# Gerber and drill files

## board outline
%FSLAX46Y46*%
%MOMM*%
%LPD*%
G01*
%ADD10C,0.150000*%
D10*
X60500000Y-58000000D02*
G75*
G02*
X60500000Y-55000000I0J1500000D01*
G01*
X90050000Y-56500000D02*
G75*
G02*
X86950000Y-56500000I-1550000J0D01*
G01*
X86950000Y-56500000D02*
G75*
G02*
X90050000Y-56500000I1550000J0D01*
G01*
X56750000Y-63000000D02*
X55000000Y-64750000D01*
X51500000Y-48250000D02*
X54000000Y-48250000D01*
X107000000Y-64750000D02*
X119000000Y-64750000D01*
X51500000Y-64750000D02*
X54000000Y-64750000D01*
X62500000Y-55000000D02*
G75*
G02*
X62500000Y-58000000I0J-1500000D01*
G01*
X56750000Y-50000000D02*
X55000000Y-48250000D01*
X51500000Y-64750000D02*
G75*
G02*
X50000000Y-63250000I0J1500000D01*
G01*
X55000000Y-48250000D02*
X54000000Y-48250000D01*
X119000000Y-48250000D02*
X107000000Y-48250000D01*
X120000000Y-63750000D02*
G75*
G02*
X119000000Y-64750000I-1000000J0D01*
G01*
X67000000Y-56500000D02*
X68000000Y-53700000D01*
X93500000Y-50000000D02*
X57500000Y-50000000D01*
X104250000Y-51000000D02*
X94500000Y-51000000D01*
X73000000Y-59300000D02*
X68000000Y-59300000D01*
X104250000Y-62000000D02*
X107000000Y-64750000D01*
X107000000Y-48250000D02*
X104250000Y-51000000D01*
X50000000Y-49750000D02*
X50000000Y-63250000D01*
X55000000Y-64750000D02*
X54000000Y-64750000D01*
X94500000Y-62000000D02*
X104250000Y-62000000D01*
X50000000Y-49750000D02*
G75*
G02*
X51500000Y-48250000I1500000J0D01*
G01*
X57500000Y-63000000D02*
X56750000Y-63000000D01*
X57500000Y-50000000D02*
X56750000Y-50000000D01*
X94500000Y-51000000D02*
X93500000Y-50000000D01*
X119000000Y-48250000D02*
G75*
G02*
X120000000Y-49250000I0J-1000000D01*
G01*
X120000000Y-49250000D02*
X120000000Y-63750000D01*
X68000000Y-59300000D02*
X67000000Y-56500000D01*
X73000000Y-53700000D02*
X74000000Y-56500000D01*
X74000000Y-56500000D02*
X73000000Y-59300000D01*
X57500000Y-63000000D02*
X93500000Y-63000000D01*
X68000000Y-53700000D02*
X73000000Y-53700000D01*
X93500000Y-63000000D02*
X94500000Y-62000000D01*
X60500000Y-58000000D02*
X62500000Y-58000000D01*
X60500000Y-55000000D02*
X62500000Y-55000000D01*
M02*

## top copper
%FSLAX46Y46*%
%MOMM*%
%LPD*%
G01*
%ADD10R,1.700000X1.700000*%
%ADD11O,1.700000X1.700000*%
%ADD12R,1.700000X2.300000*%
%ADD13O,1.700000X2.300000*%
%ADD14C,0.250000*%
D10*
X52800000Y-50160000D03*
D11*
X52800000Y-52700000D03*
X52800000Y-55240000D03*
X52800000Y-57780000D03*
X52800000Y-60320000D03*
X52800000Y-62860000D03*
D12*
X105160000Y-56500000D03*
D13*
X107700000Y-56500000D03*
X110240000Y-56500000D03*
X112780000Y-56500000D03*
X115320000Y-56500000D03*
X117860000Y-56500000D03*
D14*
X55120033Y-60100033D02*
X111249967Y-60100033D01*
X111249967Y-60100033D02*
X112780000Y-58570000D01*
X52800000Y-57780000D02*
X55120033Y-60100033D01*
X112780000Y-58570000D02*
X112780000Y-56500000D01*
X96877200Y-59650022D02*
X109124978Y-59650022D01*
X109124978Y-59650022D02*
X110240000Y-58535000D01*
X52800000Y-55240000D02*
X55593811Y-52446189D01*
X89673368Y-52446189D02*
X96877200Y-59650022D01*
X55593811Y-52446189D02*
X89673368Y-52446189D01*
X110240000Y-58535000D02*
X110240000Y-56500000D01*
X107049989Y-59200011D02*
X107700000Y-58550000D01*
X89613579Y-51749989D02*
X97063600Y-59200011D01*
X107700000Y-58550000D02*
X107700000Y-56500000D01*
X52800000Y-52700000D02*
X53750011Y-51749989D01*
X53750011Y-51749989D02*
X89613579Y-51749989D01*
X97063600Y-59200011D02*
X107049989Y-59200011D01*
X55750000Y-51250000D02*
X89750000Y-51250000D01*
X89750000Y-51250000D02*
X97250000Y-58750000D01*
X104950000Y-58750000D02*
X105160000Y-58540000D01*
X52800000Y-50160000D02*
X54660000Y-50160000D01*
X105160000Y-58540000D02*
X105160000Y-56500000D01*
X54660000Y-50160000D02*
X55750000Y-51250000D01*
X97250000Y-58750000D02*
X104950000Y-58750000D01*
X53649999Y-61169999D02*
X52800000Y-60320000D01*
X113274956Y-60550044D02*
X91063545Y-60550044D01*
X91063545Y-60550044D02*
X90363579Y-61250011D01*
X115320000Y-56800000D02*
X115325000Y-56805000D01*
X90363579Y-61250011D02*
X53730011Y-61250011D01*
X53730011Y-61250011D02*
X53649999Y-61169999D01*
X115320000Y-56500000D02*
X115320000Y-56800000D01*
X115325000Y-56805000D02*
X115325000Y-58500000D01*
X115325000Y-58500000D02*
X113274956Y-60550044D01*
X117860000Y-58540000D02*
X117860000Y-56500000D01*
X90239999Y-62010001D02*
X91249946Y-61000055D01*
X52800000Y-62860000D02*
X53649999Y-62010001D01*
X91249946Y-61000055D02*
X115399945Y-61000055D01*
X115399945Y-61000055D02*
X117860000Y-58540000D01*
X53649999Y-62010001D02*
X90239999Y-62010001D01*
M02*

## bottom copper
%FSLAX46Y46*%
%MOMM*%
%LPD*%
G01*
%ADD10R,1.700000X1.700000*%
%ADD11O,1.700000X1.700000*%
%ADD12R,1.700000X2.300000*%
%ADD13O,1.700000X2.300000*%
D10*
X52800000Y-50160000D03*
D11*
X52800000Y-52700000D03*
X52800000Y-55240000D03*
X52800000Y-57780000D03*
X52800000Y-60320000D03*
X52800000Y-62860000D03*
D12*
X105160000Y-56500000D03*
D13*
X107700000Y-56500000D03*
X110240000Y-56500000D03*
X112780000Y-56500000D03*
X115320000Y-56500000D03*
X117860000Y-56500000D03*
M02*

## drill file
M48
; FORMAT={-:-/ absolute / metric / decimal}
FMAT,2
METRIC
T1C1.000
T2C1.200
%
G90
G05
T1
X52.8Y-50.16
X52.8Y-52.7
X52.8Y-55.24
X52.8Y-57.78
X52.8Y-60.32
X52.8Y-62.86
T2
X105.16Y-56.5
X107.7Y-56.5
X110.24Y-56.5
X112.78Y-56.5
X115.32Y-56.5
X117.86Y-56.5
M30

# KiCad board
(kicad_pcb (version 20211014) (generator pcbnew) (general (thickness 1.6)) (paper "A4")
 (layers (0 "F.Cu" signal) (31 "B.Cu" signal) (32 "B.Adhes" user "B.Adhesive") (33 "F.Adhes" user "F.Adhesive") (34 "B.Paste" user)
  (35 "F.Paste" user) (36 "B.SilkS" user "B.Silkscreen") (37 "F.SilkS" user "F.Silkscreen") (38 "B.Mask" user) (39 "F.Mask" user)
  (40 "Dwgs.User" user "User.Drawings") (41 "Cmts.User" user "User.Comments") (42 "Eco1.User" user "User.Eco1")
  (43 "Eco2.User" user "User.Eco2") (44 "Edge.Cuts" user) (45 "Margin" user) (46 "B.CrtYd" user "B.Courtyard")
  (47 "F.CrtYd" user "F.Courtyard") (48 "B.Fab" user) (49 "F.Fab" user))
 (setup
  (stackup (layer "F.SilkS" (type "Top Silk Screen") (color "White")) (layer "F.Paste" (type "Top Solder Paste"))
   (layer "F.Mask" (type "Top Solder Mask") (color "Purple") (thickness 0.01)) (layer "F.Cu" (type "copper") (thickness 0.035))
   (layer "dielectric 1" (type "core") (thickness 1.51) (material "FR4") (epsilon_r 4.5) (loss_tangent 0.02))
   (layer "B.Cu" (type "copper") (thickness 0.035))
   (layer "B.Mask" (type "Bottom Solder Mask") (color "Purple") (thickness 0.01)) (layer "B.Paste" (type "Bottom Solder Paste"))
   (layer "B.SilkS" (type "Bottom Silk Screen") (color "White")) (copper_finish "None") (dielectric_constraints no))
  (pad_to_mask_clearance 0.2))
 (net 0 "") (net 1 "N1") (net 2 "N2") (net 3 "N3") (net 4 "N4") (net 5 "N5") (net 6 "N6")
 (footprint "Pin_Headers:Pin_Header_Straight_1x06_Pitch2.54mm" (layer "F.Cu") (at 52.8 50.16)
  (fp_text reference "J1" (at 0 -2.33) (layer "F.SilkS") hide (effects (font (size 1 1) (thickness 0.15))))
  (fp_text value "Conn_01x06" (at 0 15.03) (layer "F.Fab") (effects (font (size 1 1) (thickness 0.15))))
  (pad "1" thru_hole rect locked (at 0 0) (size 1.7 1.7) (drill 1) (layers *.Cu *.Mask) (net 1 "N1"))
  (pad "2" thru_hole oval locked (at 0 2.54) (size 1.7 1.7) (drill 1) (layers *.Cu *.Mask) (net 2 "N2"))
  (pad "3" thru_hole oval locked (at 0 5.08) (size 1.7 1.7) (drill 1) (layers *.Cu *.Mask) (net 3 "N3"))
  (pad "4" thru_hole oval locked (at 0 7.62) (size 1.7 1.7) (drill 1) (layers *.Cu *.Mask) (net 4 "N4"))
  (pad "5" thru_hole oval locked (at 0 10.16) (size 1.7 1.7) (drill 1) (layers *.Cu *.Mask) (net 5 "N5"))
  (pad "6" thru_hole oval locked (at 0 12.7) (size 1.7 1.7) (drill 1) (layers *.Cu *.Mask) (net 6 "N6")))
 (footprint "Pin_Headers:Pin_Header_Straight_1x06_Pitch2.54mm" (layer "F.Cu") (at 105.16 56.5 90)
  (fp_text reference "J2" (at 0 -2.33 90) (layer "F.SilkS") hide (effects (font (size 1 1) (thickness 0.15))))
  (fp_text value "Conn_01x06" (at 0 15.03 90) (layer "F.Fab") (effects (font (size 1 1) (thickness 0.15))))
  (pad "1" thru_hole rect locked (at 0 0 90) (size 2.3 1.7) (drill 1.2) (layers *.Cu *.Mask) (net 1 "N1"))
  (pad "2" thru_hole oval locked (at 0 2.54 90) (size 2.3 1.7) (drill 1.2) (layers *.Cu *.Mask) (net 2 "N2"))
  (pad "3" thru_hole oval locked (at 0 5.08 90) (size 2.3 1.7) (drill 1.2) (layers *.Cu *.Mask) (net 3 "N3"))
  (pad "4" thru_hole oval locked (at 0 7.62 90) (size 2.3 1.7) (drill 1.2) (layers *.Cu *.Mask) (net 4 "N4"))
  (pad "5" thru_hole oval locked (at 0 10.16 90) (size 2.3 1.7) (drill 1.2) (layers *.Cu *.Mask) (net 5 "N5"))
  (pad "6" thru_hole oval locked (at 0 12.7 90) (size 2.3 1.7) (drill 1.2) (layers *.Cu *.Mask) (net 6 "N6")))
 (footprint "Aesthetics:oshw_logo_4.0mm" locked (layer "F.Cu") (at 99.695 56.515 -90)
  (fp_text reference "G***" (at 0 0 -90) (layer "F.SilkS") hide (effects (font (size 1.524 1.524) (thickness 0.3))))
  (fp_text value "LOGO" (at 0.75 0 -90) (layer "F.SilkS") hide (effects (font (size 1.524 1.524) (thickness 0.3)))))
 (gr_arc (start 60.5 58) (mid 59 56.5) (end 60.5 55) (layer "Edge.Cuts") (width 0.15))
 (gr_arc (start 90.05 56.5) (mid 88.5 58.05) (end 86.95 56.5) (layer "Edge.Cuts") (width 0.15))
 (gr_arc (start 86.95 56.5) (mid 88.5 54.95) (end 90.05 56.5) (layer "Edge.Cuts") (width 0.15))
 (gr_line (start 56.75 63) (end 55 64.75) (layer "Edge.Cuts") (width 0.15))
 (gr_line (start 51.5 48.25) (end 54 48.25) (layer "Edge.Cuts") (width 0.15))
 (gr_line (start 107 64.75) (end 119 64.75) (layer "Edge.Cuts") (width 0.15))
 (gr_line (start 51.5 64.75) (end 54 64.75) (layer "Edge.Cuts") (width 0.15))
 (gr_arc (start 62.5 55) (mid 64 56.5) (end 62.5 58) (layer "Edge.Cuts") (width 0.15))
 (gr_line (start 56.75 50) (end 55 48.25) (layer "Edge.Cuts") (width 0.15))
 (gr_arc (start 51.5 64.75) (mid 50.43934 64.31066) (end 50 63.25) (layer "Edge.Cuts") (width 0.15))
 (gr_line (start 55 48.25) (end 54 48.25) (layer "Edge.Cuts") (width 0.15))
 (gr_line (start 119 48.25) (end 107 48.25) (layer "Edge.Cuts") (width 0.15))
 (gr_arc (start 120 63.75) (mid 119.707107 64.457107) (end 119 64.75) (layer "Edge.Cuts") (width 0.15))
 (gr_line (start 67 56.5) (end 68 53.7) (layer "Edge.Cuts") (width 0.15))
 (gr_line (start 93.5 50) (end 57.5 50) (layer "Edge.Cuts") (width 0.15))
 (gr_line (start 104.25 51) (end 94.5 51) (layer "Edge.Cuts") (width 0.15))
 (gr_line (start 73 59.3) (end 68 59.3) (layer "Edge.Cuts") (width 0.15))
 (gr_line (start 104.25 62) (end 107 64.75) (layer "Edge.Cuts") (width 0.15))
 (gr_line (start 107 48.25) (end 104.25 51) (layer "Edge.Cuts") (width 0.15))
 (gr_line (start 50 49.75) (end 50 63.25) (layer "Edge.Cuts") (width 0.15))
 (gr_line (start 55 64.75) (end 54 64.75) (layer "Edge.Cuts") (width 0.15))
 (gr_line (start 94.5 62) (end 104.25 62) (layer "Edge.Cuts") (width 0.15))
 (gr_arc (start 50 49.75) (mid 50.43934 48.68934) (end 51.5 48.25) (layer "Edge.Cuts") (width 0.15))
 (gr_line (start 57.5 63) (end 56.75 63) (layer "Edge.Cuts") (width 0.15))
 (gr_line (start 57.5 50) (end 56.75 50) (layer "Edge.Cuts") (width 0.15))
 (gr_line (start 94.5 51) (end 93.5 50) (layer "Edge.Cuts") (width 0.15))
 (gr_arc (start 119 48.25) (mid 119.707107 48.542893) (end 120 49.25) (layer "Edge.Cuts") (width 0.15))
 (gr_line (start 120 49.25) (end 120 63.75) (layer "Edge.Cuts") (width 0.15))
 (gr_line (start 68 59.3) (end 67 56.5) (layer "Edge.Cuts") (width 0.15))
 (gr_line (start 73 53.7) (end 74 56.5) (layer "Edge.Cuts") (width 0.15))
 (gr_line (start 74 56.5) (end 73 59.3) (layer "Edge.Cuts") (width 0.15))
 (gr_line (start 57.5 63) (end 93.5 63) (layer "Edge.Cuts") (width 0.15))
 (gr_line (start 68 53.7) (end 73 53.7) (layer "Edge.Cuts") (width 0.15))
 (gr_line (start 93.5 63) (end 94.5 62) (layer "Edge.Cuts") (width 0.15))
 (gr_line (start 60.5 58) (end 62.5 58) (layer "Edge.Cuts") (width 0.15))
 (gr_line (start 60.5 55) (end 62.5 55) (layer "Edge.Cuts") (width 0.15))
 (segment (start 55.120033 60.100033) (end 111.249967 60.100033) (width 0.25) (layer "F.Cu") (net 4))
 (segment (start 111.249967 60.100033) (end 112.78 58.57) (width 0.25) (layer "F.Cu") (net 4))
 (segment (start 52.8 57.78) (end 55.120033 60.100033) (width 0.25) (layer "F.Cu") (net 4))
 (segment (start 112.78 58.57) (end 112.78 56.5) (width 0.25) (layer "F.Cu") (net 4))
 (segment (start 96.8772 59.650022) (end 109.124978 59.650022) (width 0.25) (layer "F.Cu") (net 3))
 (segment (start 109.124978 59.650022) (end 110.24 58.535) (width 0.25) (layer "F.Cu") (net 3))
 (segment (start 52.8 55.24) (end 55.593811 52.446189) (width 0.25) (layer "F.Cu") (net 3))
 (segment (start 89.673368 52.446189) (end 96.8772 59.650022) (width 0.25) (layer "F.Cu") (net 3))
 (segment (start 55.593811 52.446189) (end 89.673368 52.446189) (width 0.25) (layer "F.Cu") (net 3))
 (segment (start 110.24 58.535) (end 110.24 56.5) (width 0.25) (layer "F.Cu") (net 3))
 (segment (start 107.049989 59.200011) (end 107.7 58.55) (width 0.25) (layer "F.Cu") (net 2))
 (segment (start 89.613579 51.749989) (end 97.0636 59.200011) (width 0.25) (layer "F.Cu") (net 2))
 (segment (start 107.7 58.55) (end 107.7 56.5) (width 0.25) (layer "F.Cu") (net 2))
 (segment (start 52.8 52.7) (end 53.750011 51.749989) (width 0.25) (layer "F.Cu") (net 2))
 (segment (start 53.750011 51.749989) (end 89.613579 51.749989) (width 0.25) (layer "F.Cu") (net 2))
 (segment (start 97.0636 59.200011) (end 107.049989 59.200011) (width 0.25) (layer "F.Cu") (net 2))
 (segment (start 55.75 51.25) (end 89.75 51.25) (width 0.25) (layer "F.Cu") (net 1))
 (segment (start 89.75 51.25) (end 97.25 58.75) (width 0.25) (layer "F.Cu") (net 1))
 (segment (start 104.95 58.75) (end 105.16 58.54) (width 0.25) (layer "F.Cu") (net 1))
 (segment (start 52.8 50.16) (end 54.66 50.16) (width 0.25) (layer "F.Cu") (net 1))
 (segment (start 105.16 58.54) (end 105.16 56.5) (width 0.25) (layer "F.Cu") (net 1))
 (segment (start 54.66 50.16) (end 55.75 51.25) (width 0.25) (layer "F.Cu") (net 1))
 (segment (start 97.25 58.75) (end 104.95 58.75) (width 0.25) (layer "F.Cu") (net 1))
 (segment (start 53.649999 61.169999) (end 52.8 60.32) (width 0.25) (layer "F.Cu") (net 5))
 (segment (start 113.274956 60.550044) (end 91.063545 60.550044) (width 0.25) (layer "F.Cu") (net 5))
 (segment (start 91.063545 60.550044) (end 90.363579 61.250011) (width 0.25) (layer "F.Cu") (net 5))
 (segment (start 115.32 56.8) (end 115.325 56.805) (width 0.25) (layer "F.Cu") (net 5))
 (segment (start 90.363579 61.250011) (end 53.730011 61.250011) (width 0.25) (layer "F.Cu") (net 5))
 (segment (start 53.730011 61.250011) (end 53.649999 61.169999) (width 0.25) (layer "F.Cu") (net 5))
 (segment (start 115.32 56.5) (end 115.32 56.8) (width 0.25) (layer "F.Cu") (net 5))
 (segment (start 115.325 56.805) (end 115.325 58.5) (width 0.25) (layer "F.Cu") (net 5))
 (segment (start 115.325 58.5) (end 113.274956 60.550044) (width 0.25) (layer "F.Cu") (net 5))
 (segment (start 117.86 58.54) (end 117.86 56.5) (width 0.25) (layer "F.Cu") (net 6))
 (segment (start 90.239999 62.010001) (end 91.249946 61.000055) (width 0.25) (layer "F.Cu") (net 6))
 (segment (start 52.8 62.86) (end 53.649999 62.010001) (width 0.25) (layer "F.Cu") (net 6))
 (segment (start 91.249946 61.000055) (end 115.399945 61.000055) (width 0.25) (layer "F.Cu") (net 6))
 (segment (start 115.399945 61.000055) (end 117.86 58.54) (width 0.25) (layer "F.Cu") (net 6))
 (segment (start 53.649999 62.010001) (end 90.239999 62.010001) (width 0.25) (layer "F.Cu") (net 6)))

